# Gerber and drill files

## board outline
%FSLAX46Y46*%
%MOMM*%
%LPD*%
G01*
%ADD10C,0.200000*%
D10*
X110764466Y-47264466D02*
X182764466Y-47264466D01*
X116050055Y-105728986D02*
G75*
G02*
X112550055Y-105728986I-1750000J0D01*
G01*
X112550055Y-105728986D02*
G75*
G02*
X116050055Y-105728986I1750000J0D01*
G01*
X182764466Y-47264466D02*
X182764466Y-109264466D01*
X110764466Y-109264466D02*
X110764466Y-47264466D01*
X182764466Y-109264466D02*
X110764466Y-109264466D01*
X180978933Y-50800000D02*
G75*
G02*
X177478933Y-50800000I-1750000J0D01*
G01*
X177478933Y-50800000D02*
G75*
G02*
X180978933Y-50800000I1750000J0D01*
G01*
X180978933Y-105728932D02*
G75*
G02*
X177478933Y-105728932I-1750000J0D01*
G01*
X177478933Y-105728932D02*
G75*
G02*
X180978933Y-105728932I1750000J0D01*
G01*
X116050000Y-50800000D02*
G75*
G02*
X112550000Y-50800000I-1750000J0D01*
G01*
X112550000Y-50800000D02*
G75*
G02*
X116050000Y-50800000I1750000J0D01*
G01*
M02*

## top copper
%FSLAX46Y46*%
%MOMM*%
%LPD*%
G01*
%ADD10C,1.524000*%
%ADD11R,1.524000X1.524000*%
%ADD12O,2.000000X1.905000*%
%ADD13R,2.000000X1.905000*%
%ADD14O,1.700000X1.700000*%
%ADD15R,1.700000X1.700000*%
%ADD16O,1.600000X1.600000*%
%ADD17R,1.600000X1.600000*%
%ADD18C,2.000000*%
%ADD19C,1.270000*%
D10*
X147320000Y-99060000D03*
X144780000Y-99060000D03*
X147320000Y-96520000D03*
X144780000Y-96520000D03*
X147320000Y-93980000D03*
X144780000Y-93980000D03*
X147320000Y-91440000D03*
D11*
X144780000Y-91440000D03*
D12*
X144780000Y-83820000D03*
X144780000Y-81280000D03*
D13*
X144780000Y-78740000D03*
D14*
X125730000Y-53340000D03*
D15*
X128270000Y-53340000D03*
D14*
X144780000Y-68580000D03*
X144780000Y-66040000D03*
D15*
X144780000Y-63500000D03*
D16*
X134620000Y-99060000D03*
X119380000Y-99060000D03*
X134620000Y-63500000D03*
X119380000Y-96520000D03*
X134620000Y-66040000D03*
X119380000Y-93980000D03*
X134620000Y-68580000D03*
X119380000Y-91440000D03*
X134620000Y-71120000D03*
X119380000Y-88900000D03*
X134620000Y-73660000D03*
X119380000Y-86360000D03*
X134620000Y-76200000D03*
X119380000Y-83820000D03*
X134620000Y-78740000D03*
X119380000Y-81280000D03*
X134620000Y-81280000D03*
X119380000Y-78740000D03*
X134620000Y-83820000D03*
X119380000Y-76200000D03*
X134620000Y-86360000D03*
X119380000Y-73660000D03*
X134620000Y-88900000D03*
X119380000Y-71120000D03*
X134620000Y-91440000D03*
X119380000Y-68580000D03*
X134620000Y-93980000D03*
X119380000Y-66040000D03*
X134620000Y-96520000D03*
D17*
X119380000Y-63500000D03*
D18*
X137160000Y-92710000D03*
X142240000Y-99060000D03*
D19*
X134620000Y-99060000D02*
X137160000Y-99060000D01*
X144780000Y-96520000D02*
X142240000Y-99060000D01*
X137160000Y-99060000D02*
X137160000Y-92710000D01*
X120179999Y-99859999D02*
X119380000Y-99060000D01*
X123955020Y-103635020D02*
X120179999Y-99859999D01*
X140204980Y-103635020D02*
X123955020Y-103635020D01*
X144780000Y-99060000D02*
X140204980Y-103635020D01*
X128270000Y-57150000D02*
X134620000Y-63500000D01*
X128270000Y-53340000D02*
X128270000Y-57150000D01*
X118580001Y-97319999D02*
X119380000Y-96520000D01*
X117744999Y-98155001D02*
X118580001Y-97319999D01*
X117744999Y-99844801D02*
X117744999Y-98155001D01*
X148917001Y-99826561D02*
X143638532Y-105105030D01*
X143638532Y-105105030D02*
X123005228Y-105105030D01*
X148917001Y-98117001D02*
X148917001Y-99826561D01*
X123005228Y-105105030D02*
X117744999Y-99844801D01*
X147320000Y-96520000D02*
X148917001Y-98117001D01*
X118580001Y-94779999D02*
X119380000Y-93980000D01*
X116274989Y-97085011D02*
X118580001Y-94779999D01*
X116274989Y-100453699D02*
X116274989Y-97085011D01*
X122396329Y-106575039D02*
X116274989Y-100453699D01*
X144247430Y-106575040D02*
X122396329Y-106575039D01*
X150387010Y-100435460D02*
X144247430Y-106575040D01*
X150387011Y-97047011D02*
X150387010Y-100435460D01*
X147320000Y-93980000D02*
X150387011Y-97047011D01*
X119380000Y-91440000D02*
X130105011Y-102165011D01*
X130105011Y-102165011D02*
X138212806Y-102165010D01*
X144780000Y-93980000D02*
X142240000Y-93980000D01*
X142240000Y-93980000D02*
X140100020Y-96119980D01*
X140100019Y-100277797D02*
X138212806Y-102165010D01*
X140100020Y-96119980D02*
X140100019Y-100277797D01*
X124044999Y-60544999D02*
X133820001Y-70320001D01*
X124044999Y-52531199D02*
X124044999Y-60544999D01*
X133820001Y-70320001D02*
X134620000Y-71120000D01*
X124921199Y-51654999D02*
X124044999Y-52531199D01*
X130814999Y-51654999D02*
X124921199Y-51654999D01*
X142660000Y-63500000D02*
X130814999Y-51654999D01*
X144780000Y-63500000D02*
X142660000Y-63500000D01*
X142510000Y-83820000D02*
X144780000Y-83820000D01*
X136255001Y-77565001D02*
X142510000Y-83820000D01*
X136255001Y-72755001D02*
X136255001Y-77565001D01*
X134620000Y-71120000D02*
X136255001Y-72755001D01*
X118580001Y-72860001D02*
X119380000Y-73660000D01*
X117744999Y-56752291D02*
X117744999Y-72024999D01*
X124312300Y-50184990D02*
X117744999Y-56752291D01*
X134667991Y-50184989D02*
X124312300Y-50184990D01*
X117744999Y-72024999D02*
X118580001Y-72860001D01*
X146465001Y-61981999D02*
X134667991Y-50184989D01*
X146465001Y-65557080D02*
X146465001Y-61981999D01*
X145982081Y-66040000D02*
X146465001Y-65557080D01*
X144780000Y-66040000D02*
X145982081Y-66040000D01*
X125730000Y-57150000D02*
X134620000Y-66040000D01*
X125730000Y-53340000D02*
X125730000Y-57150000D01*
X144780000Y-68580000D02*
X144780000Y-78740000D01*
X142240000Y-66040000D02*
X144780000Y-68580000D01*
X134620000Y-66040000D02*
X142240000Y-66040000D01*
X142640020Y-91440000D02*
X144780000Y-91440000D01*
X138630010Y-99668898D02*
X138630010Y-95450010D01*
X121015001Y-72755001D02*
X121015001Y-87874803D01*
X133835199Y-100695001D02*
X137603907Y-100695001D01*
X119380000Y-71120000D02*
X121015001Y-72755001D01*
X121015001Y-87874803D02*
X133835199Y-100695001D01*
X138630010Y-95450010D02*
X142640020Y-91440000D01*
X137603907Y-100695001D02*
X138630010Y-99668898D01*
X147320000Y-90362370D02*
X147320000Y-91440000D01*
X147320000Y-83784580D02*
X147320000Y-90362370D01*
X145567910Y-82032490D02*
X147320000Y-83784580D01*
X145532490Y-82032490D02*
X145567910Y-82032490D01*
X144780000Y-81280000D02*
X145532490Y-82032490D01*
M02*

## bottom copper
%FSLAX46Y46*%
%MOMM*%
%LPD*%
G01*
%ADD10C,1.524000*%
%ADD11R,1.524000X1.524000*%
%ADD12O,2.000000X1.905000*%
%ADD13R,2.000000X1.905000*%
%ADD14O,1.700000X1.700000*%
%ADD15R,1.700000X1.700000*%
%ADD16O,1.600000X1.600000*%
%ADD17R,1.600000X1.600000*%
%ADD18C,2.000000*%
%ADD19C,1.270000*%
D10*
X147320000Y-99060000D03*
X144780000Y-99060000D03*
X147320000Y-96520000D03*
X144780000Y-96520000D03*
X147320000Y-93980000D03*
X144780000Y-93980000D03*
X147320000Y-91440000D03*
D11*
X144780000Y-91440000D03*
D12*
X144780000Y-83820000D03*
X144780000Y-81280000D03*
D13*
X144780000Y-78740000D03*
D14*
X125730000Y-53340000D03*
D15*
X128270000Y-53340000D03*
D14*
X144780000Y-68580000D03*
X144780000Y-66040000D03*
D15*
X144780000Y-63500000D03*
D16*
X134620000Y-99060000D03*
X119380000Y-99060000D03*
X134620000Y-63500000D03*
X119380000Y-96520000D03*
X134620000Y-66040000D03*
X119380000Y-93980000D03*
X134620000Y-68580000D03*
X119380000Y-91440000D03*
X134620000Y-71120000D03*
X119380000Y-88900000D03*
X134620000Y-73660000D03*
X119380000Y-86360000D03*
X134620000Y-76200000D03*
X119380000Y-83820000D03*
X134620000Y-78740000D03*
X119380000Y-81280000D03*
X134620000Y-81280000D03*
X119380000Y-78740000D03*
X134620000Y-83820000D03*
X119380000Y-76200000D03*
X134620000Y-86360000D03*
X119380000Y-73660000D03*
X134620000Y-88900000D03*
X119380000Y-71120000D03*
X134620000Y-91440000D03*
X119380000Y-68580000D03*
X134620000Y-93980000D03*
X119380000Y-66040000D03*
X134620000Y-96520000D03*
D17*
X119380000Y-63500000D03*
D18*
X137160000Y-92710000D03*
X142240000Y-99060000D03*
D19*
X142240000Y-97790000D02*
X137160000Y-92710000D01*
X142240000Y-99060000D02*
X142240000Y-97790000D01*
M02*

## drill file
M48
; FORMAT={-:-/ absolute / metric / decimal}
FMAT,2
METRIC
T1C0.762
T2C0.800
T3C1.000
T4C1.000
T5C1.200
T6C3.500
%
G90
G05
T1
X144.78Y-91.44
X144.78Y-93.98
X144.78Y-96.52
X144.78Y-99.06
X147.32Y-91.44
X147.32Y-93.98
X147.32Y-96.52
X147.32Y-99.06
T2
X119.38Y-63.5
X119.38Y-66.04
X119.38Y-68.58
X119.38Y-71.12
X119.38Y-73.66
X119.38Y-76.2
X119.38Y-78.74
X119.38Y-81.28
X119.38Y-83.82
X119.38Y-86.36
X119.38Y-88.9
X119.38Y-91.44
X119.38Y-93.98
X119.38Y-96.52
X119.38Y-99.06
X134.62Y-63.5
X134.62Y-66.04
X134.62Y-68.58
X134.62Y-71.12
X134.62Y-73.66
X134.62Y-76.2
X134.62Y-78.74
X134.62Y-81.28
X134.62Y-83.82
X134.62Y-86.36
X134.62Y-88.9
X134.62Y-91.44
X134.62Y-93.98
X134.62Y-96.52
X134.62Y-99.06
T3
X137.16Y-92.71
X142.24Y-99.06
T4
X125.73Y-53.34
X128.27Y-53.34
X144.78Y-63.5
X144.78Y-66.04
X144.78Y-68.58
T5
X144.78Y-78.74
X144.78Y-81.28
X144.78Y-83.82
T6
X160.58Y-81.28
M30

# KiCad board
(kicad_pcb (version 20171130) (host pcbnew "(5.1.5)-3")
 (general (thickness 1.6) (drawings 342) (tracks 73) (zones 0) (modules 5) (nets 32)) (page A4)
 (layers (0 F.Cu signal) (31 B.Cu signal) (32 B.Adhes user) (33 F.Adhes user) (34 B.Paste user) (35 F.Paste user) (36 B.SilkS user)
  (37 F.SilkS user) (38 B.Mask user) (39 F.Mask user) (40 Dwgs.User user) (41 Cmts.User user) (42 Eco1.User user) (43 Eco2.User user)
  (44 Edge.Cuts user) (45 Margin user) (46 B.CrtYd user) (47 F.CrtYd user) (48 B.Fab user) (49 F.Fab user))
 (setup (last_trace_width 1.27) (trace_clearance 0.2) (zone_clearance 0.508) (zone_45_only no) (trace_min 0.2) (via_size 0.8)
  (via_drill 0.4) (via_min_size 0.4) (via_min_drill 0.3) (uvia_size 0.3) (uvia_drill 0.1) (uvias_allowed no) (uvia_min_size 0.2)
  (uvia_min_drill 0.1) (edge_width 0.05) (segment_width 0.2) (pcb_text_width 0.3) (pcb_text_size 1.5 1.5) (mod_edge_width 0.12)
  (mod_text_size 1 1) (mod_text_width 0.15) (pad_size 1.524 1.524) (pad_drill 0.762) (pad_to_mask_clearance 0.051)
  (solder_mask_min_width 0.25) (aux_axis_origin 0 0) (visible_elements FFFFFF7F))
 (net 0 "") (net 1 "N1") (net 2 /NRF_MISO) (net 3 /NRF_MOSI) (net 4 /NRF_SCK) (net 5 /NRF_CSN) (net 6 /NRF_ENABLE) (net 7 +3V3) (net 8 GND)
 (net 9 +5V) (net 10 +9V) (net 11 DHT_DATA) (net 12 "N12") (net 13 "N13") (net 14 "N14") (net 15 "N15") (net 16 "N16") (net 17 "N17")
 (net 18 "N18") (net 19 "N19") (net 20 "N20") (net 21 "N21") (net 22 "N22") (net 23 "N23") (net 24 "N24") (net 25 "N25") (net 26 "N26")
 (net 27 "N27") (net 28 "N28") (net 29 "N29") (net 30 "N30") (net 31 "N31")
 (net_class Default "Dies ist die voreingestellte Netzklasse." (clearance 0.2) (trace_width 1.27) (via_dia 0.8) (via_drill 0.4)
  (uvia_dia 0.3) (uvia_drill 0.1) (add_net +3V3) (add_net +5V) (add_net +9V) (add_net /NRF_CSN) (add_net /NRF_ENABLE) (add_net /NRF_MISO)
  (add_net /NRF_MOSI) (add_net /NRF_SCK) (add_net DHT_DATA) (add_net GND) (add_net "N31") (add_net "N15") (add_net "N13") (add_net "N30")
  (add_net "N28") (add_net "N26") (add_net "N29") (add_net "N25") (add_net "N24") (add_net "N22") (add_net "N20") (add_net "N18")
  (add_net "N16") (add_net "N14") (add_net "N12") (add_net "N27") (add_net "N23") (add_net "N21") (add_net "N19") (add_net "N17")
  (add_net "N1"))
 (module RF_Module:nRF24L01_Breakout (layer F.Cu) (at 144.78 91.44)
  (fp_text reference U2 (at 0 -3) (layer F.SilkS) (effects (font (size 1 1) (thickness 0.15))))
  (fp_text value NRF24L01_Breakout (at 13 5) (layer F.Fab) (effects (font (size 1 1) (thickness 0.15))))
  (pad 8 thru_hole circle (at 2.54 7.62) (size 1.524 1.524) (drill 0.762) (layers *.Cu *.Mask) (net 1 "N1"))
  (pad 7 thru_hole circle (at 0 7.62) (size 1.524 1.524) (drill 0.762) (layers *.Cu *.Mask) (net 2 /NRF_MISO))
  (pad 6 thru_hole circle (at 2.54 5.08) (size 1.524 1.524) (drill 0.762) (layers *.Cu *.Mask) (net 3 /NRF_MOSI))
  (pad 5 thru_hole circle (at 0 5.08) (size 1.524 1.524) (drill 0.762) (layers *.Cu *.Mask) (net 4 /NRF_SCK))
  (pad 4 thru_hole circle (at 2.54 2.54) (size 1.524 1.524) (drill 0.762) (layers *.Cu *.Mask) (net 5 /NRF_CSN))
  (pad 3 thru_hole circle (at 0 2.54) (size 1.524 1.524) (drill 0.762) (layers *.Cu *.Mask) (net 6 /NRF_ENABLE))
  (pad 2 thru_hole circle (at 2.54 0) (size 1.524 1.524) (drill 0.762) (layers *.Cu *.Mask) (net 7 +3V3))
  (pad 1 thru_hole rect (at 0 0) (size 1.524 1.524) (drill 0.762) (layers *.Cu *.Mask) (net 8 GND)))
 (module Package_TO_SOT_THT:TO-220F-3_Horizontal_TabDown (layer F.Cu) (at 144.78 78.74 270)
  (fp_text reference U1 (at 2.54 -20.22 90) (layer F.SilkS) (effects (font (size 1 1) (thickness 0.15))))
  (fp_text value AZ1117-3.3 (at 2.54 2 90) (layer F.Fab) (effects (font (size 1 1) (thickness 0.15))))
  (pad 3 thru_hole oval (at 5.08 0 270) (size 1.905 2) (drill 1.2) (layers *.Cu *.Mask) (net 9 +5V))
  (pad 2 thru_hole oval (at 2.54 0 270) (size 1.905 2) (drill 1.2) (layers *.Cu *.Mask) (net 7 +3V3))
  (pad 1 thru_hole rect (at 0 0 270) (size 1.905 2) (drill 1.2) (layers *.Cu *.Mask) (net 8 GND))
  (pad "" np_thru_hole oval (at 2.54 -15.8 270) (size 3.5 3.5) (drill 3.5) (layers *.Cu *.Mask)))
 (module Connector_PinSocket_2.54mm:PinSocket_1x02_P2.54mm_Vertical (layer F.Cu) (at 128.27 53.34 270)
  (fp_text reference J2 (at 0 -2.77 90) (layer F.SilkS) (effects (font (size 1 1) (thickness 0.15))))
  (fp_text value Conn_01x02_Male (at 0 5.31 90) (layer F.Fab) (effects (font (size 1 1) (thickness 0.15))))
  (pad 2 thru_hole oval (at 0 2.54 270) (size 1.7 1.7) (drill 1) (layers *.Cu *.Mask) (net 8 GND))
  (pad 1 thru_hole rect (at 0 0 270) (size 1.7 1.7) (drill 1) (layers *.Cu *.Mask) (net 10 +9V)))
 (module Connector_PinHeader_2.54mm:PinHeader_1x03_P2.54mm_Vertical (layer F.Cu) (at 144.78 63.5)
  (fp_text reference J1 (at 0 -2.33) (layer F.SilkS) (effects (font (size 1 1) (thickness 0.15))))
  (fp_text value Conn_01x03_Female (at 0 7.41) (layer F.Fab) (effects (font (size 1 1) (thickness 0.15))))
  (pad 3 thru_hole oval (at 0 5.08) (size 1.7 1.7) (drill 1) (layers *.Cu *.Mask) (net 8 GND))
  (pad 2 thru_hole oval (at 0 2.54) (size 1.7 1.7) (drill 1) (layers *.Cu *.Mask) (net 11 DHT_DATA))
  (pad 1 thru_hole rect (at 0 0) (size 1.7 1.7) (drill 1) (layers *.Cu *.Mask) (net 9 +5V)))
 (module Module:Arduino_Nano (layer F.Cu) (at 119.38 63.5)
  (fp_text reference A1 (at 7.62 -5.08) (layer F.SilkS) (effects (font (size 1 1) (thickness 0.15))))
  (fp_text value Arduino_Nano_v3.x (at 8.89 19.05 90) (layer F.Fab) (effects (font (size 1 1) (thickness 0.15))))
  (pad 16 thru_hole oval (at 15.24 35.56) (size 1.6 1.6) (drill 0.8) (layers *.Cu *.Mask) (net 4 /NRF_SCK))
  (pad 15 thru_hole oval (at 0 35.56) (size 1.6 1.6) (drill 0.8) (layers *.Cu *.Mask) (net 2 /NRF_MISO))
  (pad 30 thru_hole oval (at 15.24 0) (size 1.6 1.6) (drill 0.8) (layers *.Cu *.Mask) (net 10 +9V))
  (pad 14 thru_hole oval (at 0 33.02) (size 1.6 1.6) (drill 0.8) (layers *.Cu *.Mask) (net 3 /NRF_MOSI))
  (pad 29 thru_hole oval (at 15.24 2.54) (size 1.6 1.6) (drill 0.8) (layers *.Cu *.Mask) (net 8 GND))
  (pad 13 thru_hole oval (at 0 30.48) (size 1.6 1.6) (drill 0.8) (layers *.Cu *.Mask) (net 5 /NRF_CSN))
  (pad 28 thru_hole oval (at 15.24 5.08) (size 1.6 1.6) (drill 0.8) (layers *.Cu *.Mask) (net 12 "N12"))
  (pad 12 thru_hole oval (at 0 27.94) (size 1.6 1.6) (drill 0.8) (layers *.Cu *.Mask) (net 6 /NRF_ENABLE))
  (pad 27 thru_hole oval (at 15.24 7.62) (size 1.6 1.6) (drill 0.8) (layers *.Cu *.Mask) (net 9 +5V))
  (pad 11 thru_hole oval (at 0 25.4) (size 1.6 1.6) (drill 0.8) (layers *.Cu *.Mask) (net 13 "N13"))
  (pad 26 thru_hole oval (at 15.24 10.16) (size 1.6 1.6) (drill 0.8) (layers *.Cu *.Mask) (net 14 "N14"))
  (pad 10 thru_hole oval (at 0 22.86) (size 1.6 1.6) (drill 0.8) (layers *.Cu *.Mask) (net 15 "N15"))
  (pad 25 thru_hole oval (at 15.24 12.7) (size 1.6 1.6) (drill 0.8) (layers *.Cu *.Mask) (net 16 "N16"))
  (pad 9 thru_hole oval (at 0 20.32) (size 1.6 1.6) (drill 0.8) (layers *.Cu *.Mask) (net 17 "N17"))
  (pad 24 thru_hole oval (at 15.24 15.24) (size 1.6 1.6) (drill 0.8) (layers *.Cu *.Mask) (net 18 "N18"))
  (pad 8 thru_hole oval (at 0 17.78) (size 1.6 1.6) (drill 0.8) (layers *.Cu *.Mask) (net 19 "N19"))
  (pad 23 thru_hole oval (at 15.24 17.78) (size 1.6 1.6) (drill 0.8) (layers *.Cu *.Mask) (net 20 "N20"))
  (pad 7 thru_hole oval (at 0 15.24) (size 1.6 1.6) (drill 0.8) (layers *.Cu *.Mask) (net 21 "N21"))
  (pad 22 thru_hole oval (at 15.24 20.32) (size 1.6 1.6) (drill 0.8) (layers *.Cu *.Mask) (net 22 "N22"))
  (pad 6 thru_hole oval (at 0 12.7) (size 1.6 1.6) (drill 0.8) (layers *.Cu *.Mask) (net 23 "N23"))
  (pad 21 thru_hole oval (at 15.24 22.86) (size 1.6 1.6) (drill 0.8) (layers *.Cu *.Mask) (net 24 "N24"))
  (pad 5 thru_hole oval (at 0 10.16) (size 1.6 1.6) (drill 0.8) (layers *.Cu *.Mask) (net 11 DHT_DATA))
  (pad 20 thru_hole oval (at 15.24 25.4) (size 1.6 1.6) (drill 0.8) (layers *.Cu *.Mask) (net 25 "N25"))
  (pad 4 thru_hole oval (at 0 7.62) (size 1.6 1.6) (drill 0.8) (layers *.Cu *.Mask) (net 8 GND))
  (pad 19 thru_hole oval (at 15.24 27.94) (size 1.6 1.6) (drill 0.8) (layers *.Cu *.Mask) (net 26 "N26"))
  (pad 3 thru_hole oval (at 0 5.08) (size 1.6 1.6) (drill 0.8) (layers *.Cu *.Mask) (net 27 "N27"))
  (pad 18 thru_hole oval (at 15.24 30.48) (size 1.6 1.6) (drill 0.8) (layers *.Cu *.Mask) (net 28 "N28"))
  (pad 2 thru_hole oval (at 0 2.54) (size 1.6 1.6) (drill 0.8) (layers *.Cu *.Mask) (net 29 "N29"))
  (pad 17 thru_hole oval (at 15.24 33.02) (size 1.6 1.6) (drill 0.8) (layers *.Cu *.Mask) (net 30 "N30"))
  (pad 1 thru_hole rect (at 0 0) (size 1.6 1.6) (drill 0.8) (layers *.Cu *.Mask) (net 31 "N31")))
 (gr_line (start 110.764466 47.264466) (end 182.764466 47.264466) (layer Edge.Cuts) (width 0.2))
 (gr_circle (center 114.300055 105.728986) (end 116.050055 105.728986) (layer Edge.Cuts) (width 0.2))
 (gr_line (start 182.764466 47.264466) (end 182.764466 109.264466) (layer Edge.Cuts) (width 0.2))
 (gr_line (start 110.764466 109.264466) (end 110.764466 47.264466) (layer Edge.Cuts) (width 0.2))
 (gr_line (start 182.764466 109.264466) (end 110.764466 109.264466) (layer Edge.Cuts) (width 0.2))
 (gr_circle (center 179.228933 50.8) (end 180.978933 50.8) (layer Edge.Cuts) (width 0.2))
 (gr_circle (center 179.228933 105.728932) (end 180.978933 105.728932) (layer Edge.Cuts) (width 0.2))
 (gr_circle (center 114.3 50.8) (end 116.05 50.8) (layer Edge.Cuts) (width 0.2))
 (via (at 137.16 92.71) (size 2) (drill 1) (layers F.Cu B.Cu) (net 4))
 (segment (start 134.62 99.06) (end 137.16 99.06) (width 1.27) (layer F.Cu) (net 4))
 (via (at 142.24 99.06) (size 2) (drill 1) (layers F.Cu B.Cu) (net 4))
 (segment (start 144.78 96.52) (end 142.24 99.06) (width 1.27) (layer F.Cu) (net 4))
 (segment (start 137.16 99.06) (end 137.16 92.71) (width 1.27) (layer F.Cu) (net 4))
 (segment (start 142.24 97.79) (end 137.16 92.71) (width 1.27) (layer B.Cu) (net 4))
 (segment (start 142.24 99.06) (end 142.24 97.79) (width 1.27) (layer B.Cu) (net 4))
 (segment (start 120.179999 99.859999) (end 119.38 99.06) (width 1.27) (layer F.Cu) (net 2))
 (segment (start 123.95502 103.63502) (end 120.179999 99.859999) (width 1.27) (layer F.Cu) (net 2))
 (segment (start 140.20498 103.63502) (end 123.95502 103.63502) (width 1.27) (layer F.Cu) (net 2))
 (segment (start 144.78 99.06) (end 140.20498 103.63502) (width 1.27) (layer F.Cu) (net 2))
 (segment (start 128.27 57.15) (end 134.62 63.5) (width 1.27) (layer F.Cu) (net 10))
 (segment (start 128.27 53.34) (end 128.27 57.15) (width 1.27) (layer F.Cu) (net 10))
 (segment (start 118.580001 97.319999) (end 119.38 96.52) (width 1.27) (layer F.Cu) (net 3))
 (segment (start 117.744999 98.155001) (end 118.580001 97.319999) (width 1.27) (layer F.Cu) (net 3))
 (segment (start 117.744999 99.844801) (end 117.744999 98.155001) (width 1.27) (layer F.Cu) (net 3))
 (segment (start 148.917001 99.826561) (end 143.638532 105.10503) (width 1.27) (layer F.Cu) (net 3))
 (segment (start 143.638532 105.10503) (end 123.005228 105.10503) (width 1.27) (layer F.Cu) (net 3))
 (segment (start 148.917001 98.117001) (end 148.917001 99.826561) (width 1.27) (layer F.Cu) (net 3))
 (segment (start 123.005228 105.10503) (end 117.744999 99.844801) (width 1.27) (layer F.Cu) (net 3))
 (segment (start 147.32 96.52) (end 148.917001 98.117001) (width 1.27) (layer F.Cu) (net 3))
 (segment (start 118.580001 94.779999) (end 119.38 93.98) (width 1.27) (layer F.Cu) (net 5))
 (segment (start 116.274989 97.085011) (end 118.580001 94.779999) (width 1.27) (layer F.Cu) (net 5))
 (segment (start 116.274989 100.453699) (end 116.274989 97.085011) (width 1.27) (layer F.Cu) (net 5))
 (segment (start 122.396329 106.575039) (end 116.274989 100.453699) (width 1.27) (layer F.Cu) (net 5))
 (segment (start 144.24743 106.57504) (end 122.396329 106.575039) (width 1.27) (layer F.Cu) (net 5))
 (segment (start 150.38701 100.43546) (end 144.24743 106.57504) (width 1.27) (layer F.Cu) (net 5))
 (segment (start 150.387011 97.047011) (end 150.38701 100.43546) (width 1.27) (layer F.Cu) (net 5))
 (segment (start 147.32 93.98) (end 150.387011 97.047011) (width 1.27) (layer F.Cu) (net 5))
 (segment (start 119.38 91.44) (end 130.105011 102.165011) (width 1.27) (layer F.Cu) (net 6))
 (segment (start 130.105011 102.165011) (end 138.212806 102.16501) (width 1.27) (layer F.Cu) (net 6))
 (segment (start 144.78 93.98) (end 142.24 93.98) (width 1.27) (layer F.Cu) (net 6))
 (segment (start 142.24 93.98) (end 140.10002 96.11998) (width 1.27) (layer F.Cu) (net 6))
 (segment (start 140.100019 100.277797) (end 138.212806 102.16501) (width 1.27) (layer F.Cu) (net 6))
 (segment (start 140.10002 96.11998) (end 140.100019 100.277797) (width 1.27) (layer F.Cu) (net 6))
 (segment (start 124.044999 60.544999) (end 133.820001 70.320001) (width 1.27) (layer F.Cu) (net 9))
 (segment (start 124.044999 52.531199) (end 124.044999 60.544999) (width 1.27) (layer F.Cu) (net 9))
 (segment (start 133.820001 70.320001) (end 134.62 71.12) (width 1.27) (layer F.Cu) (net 9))
 (segment (start 124.921199 51.654999) (end 124.044999 52.531199) (width 1.27) (layer F.Cu) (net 9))
 (segment (start 130.814999 51.654999) (end 124.921199 51.654999) (width 1.27) (layer F.Cu) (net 9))
 (segment (start 142.66 63.5) (end 130.814999 51.654999) (width 1.27) (layer F.Cu) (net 9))
 (segment (start 144.78 63.5) (end 142.66 63.5) (width 1.27) (layer F.Cu) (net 9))
 (segment (start 142.51 83.82) (end 144.78 83.82) (width 1.27) (layer F.Cu) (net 9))
 (segment (start 136.255001 77.565001) (end 142.51 83.82) (width 1.27) (layer F.Cu) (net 9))
 (segment (start 136.255001 72.755001) (end 136.255001 77.565001) (width 1.27) (layer F.Cu) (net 9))
 (segment (start 134.62 71.12) (end 136.255001 72.755001) (width 1.27) (layer F.Cu) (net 9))
 (segment (start 118.580001 72.860001) (end 119.38 73.66) (width 1.27) (layer F.Cu) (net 11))
 (segment (start 117.744999 56.752291) (end 117.744999 72.024999) (width 1.27) (layer F.Cu) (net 11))
 (segment (start 124.3123 50.18499) (end 117.744999 56.752291) (width 1.27) (layer F.Cu) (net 11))
 (segment (start 134.667991 50.184989) (end 124.3123 50.18499) (width 1.27) (layer F.Cu) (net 11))
 (segment (start 117.744999 72.024999) (end 118.580001 72.860001) (width 1.27) (layer F.Cu) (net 11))
 (segment (start 146.465001 61.981999) (end 134.667991 50.184989) (width 1.27) (layer F.Cu) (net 11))
 (segment (start 146.465001 65.55708) (end 146.465001 61.981999) (width 1.27) (layer F.Cu) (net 11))
 (segment (start 145.982081 66.04) (end 146.465001 65.55708) (width 1.27) (layer F.Cu) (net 11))
 (segment (start 144.78 66.04) (end 145.982081 66.04) (width 1.27) (layer F.Cu) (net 11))
 (segment (start 125.73 57.15) (end 134.62 66.04) (width 1.27) (layer F.Cu) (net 8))
 (segment (start 125.73 53.34) (end 125.73 57.15) (width 1.27) (layer F.Cu) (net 8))
 (segment (start 144.78 68.58) (end 144.78 78.74) (width 1.27) (layer F.Cu) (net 8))
 (segment (start 142.24 66.04) (end 144.78 68.58) (width 1.27) (layer F.Cu) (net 8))
 (segment (start 134.62 66.04) (end 142.24 66.04) (width 1.27) (layer F.Cu) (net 8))
 (segment (start 142.64002 91.44) (end 144.78 91.44) (width 1.27) (layer F.Cu) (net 8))
 (segment (start 138.63001 99.668898) (end 138.63001 95.45001) (width 1.27) (layer F.Cu) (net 8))
 (segment (start 121.015001 72.755001) (end 121.015001 87.874803) (width 1.27) (layer F.Cu) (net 8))
 (segment (start 133.835199 100.695001) (end 137.603907 100.695001) (width 1.27) (layer F.Cu) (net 8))
 (segment (start 119.38 71.12) (end 121.015001 72.755001) (width 1.27) (layer F.Cu) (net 8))
 (segment (start 121.015001 87.874803) (end 133.835199 100.695001) (width 1.27) (layer F.Cu) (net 8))
 (segment (start 138.63001 95.45001) (end 142.64002 91.44) (width 1.27) (layer F.Cu) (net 8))
 (segment (start 137.603907 100.695001) (end 138.63001 99.668898) (width 1.27) (layer F.Cu) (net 8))
 (segment (start 147.32 90.36237) (end 147.32 91.44) (width 1.27) (layer F.Cu) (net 7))
 (segment (start 147.32 83.78458) (end 147.32 90.36237) (width 1.27) (layer F.Cu) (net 7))
 (segment (start 145.56791 82.03249) (end 147.32 83.78458) (width 1.27) (layer F.Cu) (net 7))
 (segment (start 145.53249 82.03249) (end 145.56791 82.03249) (width 1.27) (layer F.Cu) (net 7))
 (segment (start 144.78 81.28) (end 145.53249 82.03249) (width 1.27) (layer F.Cu) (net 7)))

